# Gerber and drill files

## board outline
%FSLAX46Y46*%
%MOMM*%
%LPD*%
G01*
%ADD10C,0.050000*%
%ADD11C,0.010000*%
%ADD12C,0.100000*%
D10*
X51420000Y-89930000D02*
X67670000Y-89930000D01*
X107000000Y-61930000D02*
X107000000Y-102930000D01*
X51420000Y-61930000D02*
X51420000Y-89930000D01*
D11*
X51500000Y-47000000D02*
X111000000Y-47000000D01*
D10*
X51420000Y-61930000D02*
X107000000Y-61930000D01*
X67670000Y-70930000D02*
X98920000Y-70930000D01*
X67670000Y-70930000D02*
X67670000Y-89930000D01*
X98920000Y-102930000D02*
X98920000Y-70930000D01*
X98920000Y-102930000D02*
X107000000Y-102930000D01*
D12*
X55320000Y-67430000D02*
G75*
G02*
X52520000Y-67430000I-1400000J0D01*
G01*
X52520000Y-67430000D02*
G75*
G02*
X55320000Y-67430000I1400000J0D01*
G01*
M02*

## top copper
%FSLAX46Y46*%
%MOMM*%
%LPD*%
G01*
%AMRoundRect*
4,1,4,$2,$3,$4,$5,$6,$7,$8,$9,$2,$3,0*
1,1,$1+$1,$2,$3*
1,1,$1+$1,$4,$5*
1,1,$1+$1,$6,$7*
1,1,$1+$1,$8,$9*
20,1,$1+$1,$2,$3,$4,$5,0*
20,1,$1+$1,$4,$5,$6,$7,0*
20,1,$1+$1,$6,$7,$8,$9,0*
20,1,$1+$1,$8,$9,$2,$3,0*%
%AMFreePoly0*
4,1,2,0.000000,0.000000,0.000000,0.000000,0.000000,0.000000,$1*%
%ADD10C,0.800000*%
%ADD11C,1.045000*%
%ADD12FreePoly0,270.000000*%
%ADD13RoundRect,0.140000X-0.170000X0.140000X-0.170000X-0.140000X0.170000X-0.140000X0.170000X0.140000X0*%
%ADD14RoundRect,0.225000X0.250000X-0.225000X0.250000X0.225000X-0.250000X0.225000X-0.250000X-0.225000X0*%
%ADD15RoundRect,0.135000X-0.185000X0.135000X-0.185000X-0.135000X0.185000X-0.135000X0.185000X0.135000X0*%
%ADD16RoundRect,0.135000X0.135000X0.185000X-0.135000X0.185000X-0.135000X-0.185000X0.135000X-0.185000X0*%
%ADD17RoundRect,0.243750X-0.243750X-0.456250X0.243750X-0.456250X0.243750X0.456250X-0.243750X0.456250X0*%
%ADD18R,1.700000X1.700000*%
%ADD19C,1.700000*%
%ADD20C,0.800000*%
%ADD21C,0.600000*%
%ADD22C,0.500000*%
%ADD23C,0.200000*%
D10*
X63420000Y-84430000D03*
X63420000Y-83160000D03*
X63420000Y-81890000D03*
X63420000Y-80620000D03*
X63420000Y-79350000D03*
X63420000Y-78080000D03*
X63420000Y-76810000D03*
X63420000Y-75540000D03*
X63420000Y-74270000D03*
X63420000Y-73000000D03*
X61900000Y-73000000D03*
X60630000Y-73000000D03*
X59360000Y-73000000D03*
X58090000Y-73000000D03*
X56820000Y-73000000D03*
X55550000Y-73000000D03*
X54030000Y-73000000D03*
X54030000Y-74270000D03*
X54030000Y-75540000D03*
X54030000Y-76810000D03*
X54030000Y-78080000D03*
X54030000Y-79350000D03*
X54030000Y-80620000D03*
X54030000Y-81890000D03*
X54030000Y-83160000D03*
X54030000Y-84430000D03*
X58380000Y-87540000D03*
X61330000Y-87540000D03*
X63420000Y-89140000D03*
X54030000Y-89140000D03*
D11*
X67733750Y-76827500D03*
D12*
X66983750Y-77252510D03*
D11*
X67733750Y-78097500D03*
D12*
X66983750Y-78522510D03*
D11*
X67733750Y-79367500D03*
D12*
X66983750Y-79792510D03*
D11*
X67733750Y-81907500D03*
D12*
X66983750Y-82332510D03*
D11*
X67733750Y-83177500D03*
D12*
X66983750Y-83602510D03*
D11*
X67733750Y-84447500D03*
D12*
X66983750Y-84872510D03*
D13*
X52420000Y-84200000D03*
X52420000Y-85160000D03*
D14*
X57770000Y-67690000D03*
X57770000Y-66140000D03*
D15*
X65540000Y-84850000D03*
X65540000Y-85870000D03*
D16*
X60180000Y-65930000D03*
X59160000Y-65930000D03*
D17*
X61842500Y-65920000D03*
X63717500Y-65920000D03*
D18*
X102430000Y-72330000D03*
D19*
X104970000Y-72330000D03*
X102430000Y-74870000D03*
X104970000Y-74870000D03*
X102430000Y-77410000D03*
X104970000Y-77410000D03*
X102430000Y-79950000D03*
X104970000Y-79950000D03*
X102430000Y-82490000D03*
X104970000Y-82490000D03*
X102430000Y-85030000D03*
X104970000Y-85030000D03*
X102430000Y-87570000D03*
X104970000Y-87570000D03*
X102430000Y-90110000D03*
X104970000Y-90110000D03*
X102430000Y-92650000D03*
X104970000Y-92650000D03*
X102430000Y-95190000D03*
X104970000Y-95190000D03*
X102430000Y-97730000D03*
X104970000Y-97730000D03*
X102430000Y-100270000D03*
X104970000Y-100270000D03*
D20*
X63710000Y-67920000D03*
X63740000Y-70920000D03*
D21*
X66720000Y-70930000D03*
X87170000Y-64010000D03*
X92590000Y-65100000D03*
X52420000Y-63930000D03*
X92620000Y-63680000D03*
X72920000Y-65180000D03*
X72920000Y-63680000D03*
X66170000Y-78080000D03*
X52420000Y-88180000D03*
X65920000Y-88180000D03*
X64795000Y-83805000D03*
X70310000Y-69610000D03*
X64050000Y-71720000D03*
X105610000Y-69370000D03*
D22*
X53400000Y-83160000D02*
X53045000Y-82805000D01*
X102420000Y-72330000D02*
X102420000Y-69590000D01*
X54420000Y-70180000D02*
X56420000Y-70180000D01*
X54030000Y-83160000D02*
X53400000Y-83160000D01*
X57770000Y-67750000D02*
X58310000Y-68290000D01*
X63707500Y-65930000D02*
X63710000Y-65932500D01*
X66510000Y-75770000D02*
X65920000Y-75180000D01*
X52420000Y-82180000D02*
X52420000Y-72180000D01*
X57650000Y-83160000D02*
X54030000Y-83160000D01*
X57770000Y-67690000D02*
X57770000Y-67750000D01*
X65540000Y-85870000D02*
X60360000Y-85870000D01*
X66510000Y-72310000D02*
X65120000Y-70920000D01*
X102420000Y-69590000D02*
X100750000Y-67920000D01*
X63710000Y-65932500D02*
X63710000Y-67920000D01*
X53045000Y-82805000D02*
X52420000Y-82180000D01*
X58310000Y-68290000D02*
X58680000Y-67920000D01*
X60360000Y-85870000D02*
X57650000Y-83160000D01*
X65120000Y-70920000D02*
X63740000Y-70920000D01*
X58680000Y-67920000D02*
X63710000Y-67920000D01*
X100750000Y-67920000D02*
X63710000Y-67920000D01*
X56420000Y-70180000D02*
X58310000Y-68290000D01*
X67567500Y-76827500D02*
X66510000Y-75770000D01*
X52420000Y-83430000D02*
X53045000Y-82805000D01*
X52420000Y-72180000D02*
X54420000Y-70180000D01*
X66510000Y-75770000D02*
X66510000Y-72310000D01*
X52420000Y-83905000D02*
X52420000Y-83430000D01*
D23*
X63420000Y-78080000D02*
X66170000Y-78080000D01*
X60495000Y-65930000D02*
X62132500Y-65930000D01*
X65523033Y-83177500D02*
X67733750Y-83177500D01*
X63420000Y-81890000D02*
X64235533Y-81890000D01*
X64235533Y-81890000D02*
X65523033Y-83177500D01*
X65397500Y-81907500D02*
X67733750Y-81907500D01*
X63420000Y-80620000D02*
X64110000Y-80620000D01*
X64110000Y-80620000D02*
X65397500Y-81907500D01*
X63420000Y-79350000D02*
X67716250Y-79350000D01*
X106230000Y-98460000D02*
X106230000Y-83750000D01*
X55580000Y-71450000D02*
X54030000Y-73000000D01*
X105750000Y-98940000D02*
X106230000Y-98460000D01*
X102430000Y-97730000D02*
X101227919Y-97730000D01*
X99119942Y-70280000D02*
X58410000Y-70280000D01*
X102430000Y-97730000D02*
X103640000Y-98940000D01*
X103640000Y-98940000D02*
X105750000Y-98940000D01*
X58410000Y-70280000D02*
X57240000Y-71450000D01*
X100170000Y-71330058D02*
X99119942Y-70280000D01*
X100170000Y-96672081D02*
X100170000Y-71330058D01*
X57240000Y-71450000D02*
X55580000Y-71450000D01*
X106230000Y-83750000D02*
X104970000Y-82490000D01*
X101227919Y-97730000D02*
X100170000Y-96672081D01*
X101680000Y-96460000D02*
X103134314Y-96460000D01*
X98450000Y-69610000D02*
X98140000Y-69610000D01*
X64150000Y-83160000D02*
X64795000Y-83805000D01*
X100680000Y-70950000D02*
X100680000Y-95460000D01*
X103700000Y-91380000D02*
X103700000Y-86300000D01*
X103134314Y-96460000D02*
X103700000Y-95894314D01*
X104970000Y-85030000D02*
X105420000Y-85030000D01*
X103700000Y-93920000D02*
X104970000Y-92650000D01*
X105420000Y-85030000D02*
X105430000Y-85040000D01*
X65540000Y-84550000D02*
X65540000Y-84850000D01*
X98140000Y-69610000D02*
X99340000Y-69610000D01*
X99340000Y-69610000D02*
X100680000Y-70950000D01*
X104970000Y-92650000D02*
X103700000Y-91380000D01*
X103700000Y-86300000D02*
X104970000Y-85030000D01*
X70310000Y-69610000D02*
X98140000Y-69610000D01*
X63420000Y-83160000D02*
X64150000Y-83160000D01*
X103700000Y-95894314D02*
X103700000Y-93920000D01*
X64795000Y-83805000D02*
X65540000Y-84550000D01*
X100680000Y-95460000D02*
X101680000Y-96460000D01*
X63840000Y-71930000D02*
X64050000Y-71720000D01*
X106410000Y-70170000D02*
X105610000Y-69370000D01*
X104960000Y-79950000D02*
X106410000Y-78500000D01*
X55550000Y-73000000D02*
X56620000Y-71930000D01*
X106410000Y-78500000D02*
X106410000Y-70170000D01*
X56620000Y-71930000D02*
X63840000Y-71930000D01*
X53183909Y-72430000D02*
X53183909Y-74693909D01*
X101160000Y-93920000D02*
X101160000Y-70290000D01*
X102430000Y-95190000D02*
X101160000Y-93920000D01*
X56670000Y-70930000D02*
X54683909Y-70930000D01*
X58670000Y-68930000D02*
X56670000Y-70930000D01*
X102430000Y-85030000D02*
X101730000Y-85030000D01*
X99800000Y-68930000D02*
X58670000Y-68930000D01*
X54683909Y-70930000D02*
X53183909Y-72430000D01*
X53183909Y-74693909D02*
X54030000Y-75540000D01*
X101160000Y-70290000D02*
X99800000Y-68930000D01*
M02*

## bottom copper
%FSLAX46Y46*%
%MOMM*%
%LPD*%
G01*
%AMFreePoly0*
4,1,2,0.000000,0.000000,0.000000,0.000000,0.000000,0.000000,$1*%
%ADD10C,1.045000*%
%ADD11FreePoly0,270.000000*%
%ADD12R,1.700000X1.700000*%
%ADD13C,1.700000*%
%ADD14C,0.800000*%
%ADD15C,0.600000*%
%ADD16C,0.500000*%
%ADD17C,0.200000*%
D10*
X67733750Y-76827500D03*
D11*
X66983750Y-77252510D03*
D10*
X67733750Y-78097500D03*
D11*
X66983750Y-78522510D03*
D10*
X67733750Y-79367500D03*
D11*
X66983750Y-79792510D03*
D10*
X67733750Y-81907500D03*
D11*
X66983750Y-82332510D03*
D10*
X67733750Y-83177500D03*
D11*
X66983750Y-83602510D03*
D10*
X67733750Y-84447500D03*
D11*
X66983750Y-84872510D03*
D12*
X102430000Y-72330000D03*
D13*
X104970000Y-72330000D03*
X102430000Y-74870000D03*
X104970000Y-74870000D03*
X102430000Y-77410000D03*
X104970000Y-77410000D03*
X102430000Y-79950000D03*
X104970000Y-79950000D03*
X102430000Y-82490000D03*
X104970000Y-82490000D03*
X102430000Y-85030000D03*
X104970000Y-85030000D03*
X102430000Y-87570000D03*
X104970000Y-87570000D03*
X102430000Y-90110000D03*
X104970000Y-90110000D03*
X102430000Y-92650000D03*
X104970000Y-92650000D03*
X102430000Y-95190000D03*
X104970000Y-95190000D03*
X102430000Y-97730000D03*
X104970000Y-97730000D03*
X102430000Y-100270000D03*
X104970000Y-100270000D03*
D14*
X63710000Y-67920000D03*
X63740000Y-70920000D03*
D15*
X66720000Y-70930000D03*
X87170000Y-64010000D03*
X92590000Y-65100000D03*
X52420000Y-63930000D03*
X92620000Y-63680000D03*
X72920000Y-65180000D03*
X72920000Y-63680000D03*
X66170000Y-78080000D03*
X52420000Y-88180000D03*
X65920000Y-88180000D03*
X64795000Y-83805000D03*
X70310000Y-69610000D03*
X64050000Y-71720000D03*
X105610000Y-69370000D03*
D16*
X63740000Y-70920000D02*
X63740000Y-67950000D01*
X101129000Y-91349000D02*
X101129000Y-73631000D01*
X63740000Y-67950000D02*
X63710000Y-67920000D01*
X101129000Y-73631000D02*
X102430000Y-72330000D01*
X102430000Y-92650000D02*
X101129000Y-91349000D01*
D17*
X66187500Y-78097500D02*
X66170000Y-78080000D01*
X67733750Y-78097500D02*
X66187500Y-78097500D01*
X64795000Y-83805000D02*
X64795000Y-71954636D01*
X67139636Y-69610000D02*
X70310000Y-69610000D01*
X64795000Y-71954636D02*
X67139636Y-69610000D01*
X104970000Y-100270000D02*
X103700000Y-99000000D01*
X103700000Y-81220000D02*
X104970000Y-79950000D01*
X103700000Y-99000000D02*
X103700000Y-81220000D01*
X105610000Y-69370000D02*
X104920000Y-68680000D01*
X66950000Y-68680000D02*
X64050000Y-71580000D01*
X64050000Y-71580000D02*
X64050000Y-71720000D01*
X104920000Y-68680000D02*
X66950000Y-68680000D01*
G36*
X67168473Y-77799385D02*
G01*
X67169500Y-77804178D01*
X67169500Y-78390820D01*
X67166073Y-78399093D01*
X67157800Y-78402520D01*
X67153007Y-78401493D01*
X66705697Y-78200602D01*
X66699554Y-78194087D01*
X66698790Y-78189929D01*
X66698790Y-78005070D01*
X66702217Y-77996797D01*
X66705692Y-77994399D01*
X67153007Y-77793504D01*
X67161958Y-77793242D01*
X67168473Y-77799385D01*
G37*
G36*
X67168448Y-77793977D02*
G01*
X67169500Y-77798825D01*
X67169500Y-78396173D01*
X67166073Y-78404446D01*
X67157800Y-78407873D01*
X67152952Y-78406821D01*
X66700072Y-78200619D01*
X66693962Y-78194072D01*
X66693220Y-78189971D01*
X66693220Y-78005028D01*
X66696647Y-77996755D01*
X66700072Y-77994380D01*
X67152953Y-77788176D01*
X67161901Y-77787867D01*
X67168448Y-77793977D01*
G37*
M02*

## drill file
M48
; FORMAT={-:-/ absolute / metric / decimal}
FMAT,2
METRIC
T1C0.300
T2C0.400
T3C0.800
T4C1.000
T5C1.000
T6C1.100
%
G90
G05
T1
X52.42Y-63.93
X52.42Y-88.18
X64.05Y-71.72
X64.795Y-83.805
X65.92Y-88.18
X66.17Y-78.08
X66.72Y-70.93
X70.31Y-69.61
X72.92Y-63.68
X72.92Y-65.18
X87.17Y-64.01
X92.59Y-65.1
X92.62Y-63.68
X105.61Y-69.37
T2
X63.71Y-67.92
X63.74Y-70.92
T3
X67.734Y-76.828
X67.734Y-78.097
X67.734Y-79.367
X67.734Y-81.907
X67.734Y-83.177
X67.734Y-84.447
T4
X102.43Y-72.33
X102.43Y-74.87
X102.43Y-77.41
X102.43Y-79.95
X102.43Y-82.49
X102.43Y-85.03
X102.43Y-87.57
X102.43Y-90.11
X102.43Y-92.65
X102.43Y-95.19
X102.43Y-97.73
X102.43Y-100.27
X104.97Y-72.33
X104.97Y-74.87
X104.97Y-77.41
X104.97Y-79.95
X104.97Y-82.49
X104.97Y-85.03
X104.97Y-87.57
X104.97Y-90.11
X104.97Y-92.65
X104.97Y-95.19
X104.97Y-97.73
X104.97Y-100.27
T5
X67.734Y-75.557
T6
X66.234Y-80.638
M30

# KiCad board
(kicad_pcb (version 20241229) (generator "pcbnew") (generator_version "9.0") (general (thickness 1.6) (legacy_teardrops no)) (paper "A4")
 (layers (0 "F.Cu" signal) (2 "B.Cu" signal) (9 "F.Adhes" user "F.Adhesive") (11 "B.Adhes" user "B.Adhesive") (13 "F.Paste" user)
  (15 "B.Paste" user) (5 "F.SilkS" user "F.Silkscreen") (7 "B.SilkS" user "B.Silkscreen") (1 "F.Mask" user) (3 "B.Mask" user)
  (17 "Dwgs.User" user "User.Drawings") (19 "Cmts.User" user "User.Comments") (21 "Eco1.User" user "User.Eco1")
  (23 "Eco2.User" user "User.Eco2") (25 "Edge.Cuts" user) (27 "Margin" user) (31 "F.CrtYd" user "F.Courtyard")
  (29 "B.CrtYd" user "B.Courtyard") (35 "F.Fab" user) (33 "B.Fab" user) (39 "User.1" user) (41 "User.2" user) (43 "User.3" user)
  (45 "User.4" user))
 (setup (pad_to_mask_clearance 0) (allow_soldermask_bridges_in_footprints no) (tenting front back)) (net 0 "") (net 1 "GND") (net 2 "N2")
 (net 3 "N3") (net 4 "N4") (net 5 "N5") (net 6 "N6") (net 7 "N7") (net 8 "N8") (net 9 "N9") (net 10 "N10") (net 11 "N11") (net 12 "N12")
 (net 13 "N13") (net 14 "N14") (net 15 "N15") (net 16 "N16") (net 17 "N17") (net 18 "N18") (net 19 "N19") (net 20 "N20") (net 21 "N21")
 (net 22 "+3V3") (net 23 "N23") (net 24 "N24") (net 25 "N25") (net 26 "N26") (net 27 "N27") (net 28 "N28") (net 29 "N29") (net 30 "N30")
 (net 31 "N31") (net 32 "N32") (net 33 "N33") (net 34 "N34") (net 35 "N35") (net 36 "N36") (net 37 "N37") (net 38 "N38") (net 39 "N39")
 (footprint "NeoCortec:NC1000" (layer "F.Cu") (at 63.42 84.43 180)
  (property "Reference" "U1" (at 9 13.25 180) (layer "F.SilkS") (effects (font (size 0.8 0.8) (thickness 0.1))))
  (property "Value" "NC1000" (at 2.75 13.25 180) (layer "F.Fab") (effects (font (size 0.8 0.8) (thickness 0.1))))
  (pad "1" smd circle (at 0 0 180) (size 0.8 0.8) (layers "F.Cu" "F.Mask" "F.Paste") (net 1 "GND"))
  (pad "2" smd circle (at 0 1.27 180) (size 0.8 0.8) (layers "F.Cu" "F.Mask" "F.Paste") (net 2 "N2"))
  (pad "3" smd circle (at 0 2.54 180) (size 0.8 0.8) (layers "F.Cu" "F.Mask" "F.Paste") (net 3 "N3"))
  (pad "4" smd circle (at 0 3.81 180) (size 0.8 0.8) (layers "F.Cu" "F.Mask" "F.Paste") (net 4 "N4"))
  (pad "5" smd circle (at 0 5.08 180) (size 0.8 0.8) (layers "F.Cu" "F.Mask" "F.Paste") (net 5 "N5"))
  (pad "6" smd circle (at 0 6.35 180) (size 0.8 0.8) (layers "F.Cu" "F.Mask" "F.Paste") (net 1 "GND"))
  (pad "7" smd circle (at 0 7.62 180) (size 0.8 0.8) (layers "F.Cu" "F.Mask" "F.Paste") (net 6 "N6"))
  (pad "8" smd circle (at 0 8.89 180) (size 0.8 0.8) (layers "F.Cu" "F.Mask" "F.Paste") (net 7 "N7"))
  (pad "9" smd circle (at 0 10.16 180) (size 0.8 0.8) (layers "F.Cu" "F.Mask" "F.Paste") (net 1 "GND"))
  (pad "10" smd circle (at 0 11.43 180) (size 0.8 0.8) (layers "F.Cu" "F.Mask" "F.Paste") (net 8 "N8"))
  (pad "11" smd circle (at 1.52 11.43 180) (size 0.8 0.8) (layers "F.Cu" "F.Mask" "F.Paste") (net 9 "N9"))
  (pad "12" smd circle (at 2.79 11.43 180) (size 0.8 0.8) (layers "F.Cu" "F.Mask" "F.Paste") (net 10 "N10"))
  (pad "13" smd circle (at 4.06 11.43 180) (size 0.8 0.8) (layers "F.Cu" "F.Mask" "F.Paste") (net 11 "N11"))
  (pad "14" smd circle (at 5.33 11.43 180) (size 0.8 0.8) (layers "F.Cu" "F.Mask" "F.Paste") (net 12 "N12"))
  (pad "15" smd circle (at 6.6 11.43 180) (size 0.8 0.8) (layers "F.Cu" "F.Mask" "F.Paste") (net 1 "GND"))
  (pad "16" smd circle (at 7.87 11.43 180) (size 0.8 0.8) (layers "F.Cu" "F.Mask" "F.Paste") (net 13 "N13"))
  (pad "17" smd circle (at 9.39 11.43 180) (size 0.8 0.8) (layers "F.Cu" "F.Mask" "F.Paste") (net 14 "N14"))
  (pad "18" smd circle (at 9.39 10.16 180) (size 0.8 0.8) (layers "F.Cu" "F.Mask" "F.Paste") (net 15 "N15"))
  (pad "19" smd circle (at 9.39 8.89 180) (size 0.8 0.8) (layers "F.Cu" "F.Mask" "F.Paste") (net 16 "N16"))
  (pad "20" smd circle (at 9.39 7.62 180) (size 0.8 0.8) (layers "F.Cu" "F.Mask" "F.Paste") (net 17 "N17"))
  (pad "21" smd circle (at 9.39 6.35 180) (size 0.8 0.8) (layers "F.Cu" "F.Mask" "F.Paste") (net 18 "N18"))
  (pad "22" smd circle (at 9.39 5.08 180) (size 0.8 0.8) (layers "F.Cu" "F.Mask" "F.Paste") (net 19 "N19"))
  (pad "23" smd circle (at 9.39 3.81 180) (size 0.8 0.8) (layers "F.Cu" "F.Mask" "F.Paste") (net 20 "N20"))
  (pad "24" smd circle (at 9.39 2.54 180) (size 0.8 0.8) (layers "F.Cu" "F.Mask" "F.Paste") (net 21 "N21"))
  (pad "25" smd circle (at 9.39 1.27 180) (size 0.8 0.8) (layers "F.Cu" "F.Mask" "F.Paste") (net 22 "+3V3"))
  (pad "26" smd circle (at 9.39 0 180) (size 0.8 0.8) (layers "F.Cu" "F.Mask" "F.Paste") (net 1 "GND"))
  (pad "27" smd circle (at 5.04 -3.11 180) (size 0.8 0.8) (layers "F.Cu" "F.Mask" "F.Paste") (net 1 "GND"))
  (pad "28" smd circle (at 2.09 -3.11 180) (size 0.8 0.8) (layers "F.Cu" "F.Mask" "F.Paste") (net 1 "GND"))
  (pad "29" smd circle (at 0 -4.71 180) (size 0.8 0.8) (layers "F.Cu" "F.Mask" "F.Paste"))
  (pad "30" smd circle (at 9.39 -4.71 180) (size 0.8 0.8) (layers "F.Cu" "F.Mask" "F.Paste")))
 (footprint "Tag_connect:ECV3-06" (layer "F.Cu") (at 67.73375 76.8275 -90)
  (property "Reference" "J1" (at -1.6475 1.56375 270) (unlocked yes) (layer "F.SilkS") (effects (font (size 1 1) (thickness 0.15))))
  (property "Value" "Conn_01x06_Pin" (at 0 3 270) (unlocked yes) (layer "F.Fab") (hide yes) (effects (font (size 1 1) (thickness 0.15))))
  (pad "" np_thru_hole circle (at -1.27 0 270) (size 1 1) (drill 1) (layers "*.Cu" "*.Mask"))
  (pad "" np_thru_hole circle (at 3.81 1.5 270) (size 1.1 1.1) (drill 1.1) (layers "*.Cu" "*.Mask"))
  (pad "1" thru_hole circle (at 0 0 270) (size 1.045 1.045) (drill 0.8) (layers "*.Cu" "*.Mask") (remove_unused_layers no) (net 22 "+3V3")
   (solder_paste_margin -2147.483637))
  (pad "1" smd custom (at 0.42501 0.75 270) (size 0.000001 0.000001) (layers "F.Cu" "F.Mask") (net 22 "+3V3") (solder_mask_margin 0.000001)
   (options (clearance outline) (anchor circle)) (primitives))
  (pad "1" smd custom (at 0.42501 0.75 270) (size 0.000001 0.000001) (layers "B.Cu" "B.Mask") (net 22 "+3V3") (solder_mask_margin 0.000001)
   (options (clearance outline) (anchor circle)) (primitives))
  (pad "2" thru_hole circle (at 1.27 0 270) (size 1.045 1.045) (drill 0.8) (layers "*.Cu" "*.Mask") (remove_unused_layers no) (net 1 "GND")
   (solder_paste_margin -2147.483637)
   (teardrops (best_length_ratio 0.5) (max_length 1) (best_width_ratio 1) (max_width 2) (curved_edges no) (filter_ratio 0.9) (enabled yes)
    (allow_two_segments yes) (prefer_zone_connections yes)))
  (pad "2" smd custom (at 1.69501 0.75 270) (size 0.000001 0.000001) (layers "F.Cu" "F.Mask") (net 1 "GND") (solder_mask_margin 0.000001)
   (options (clearance outline) (anchor circle)) (primitives))
  (pad "2" smd custom (at 1.69501 0.75 270) (size 0.000001 0.000001) (layers "B.Cu" "B.Mask") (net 1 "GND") (solder_mask_margin 0.000001)
   (options (clearance outline) (anchor circle)) (primitives))
  (pad "3" thru_hole circle (at 2.54 0 270) (size 1.045 1.045) (drill 0.8) (layers "*.Cu" "*.Mask") (remove_unused_layers no) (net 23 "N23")
   (solder_paste_margin -2147.483637))
  (pad "3" smd custom (at 2.96501 0.75 270) (size 0.000001 0.000001) (layers "F.Cu" "F.Mask") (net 23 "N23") (solder_mask_margin 0.000001)
   (options (clearance outline) (anchor circle)) (primitives))
  (pad "3" smd custom (at 2.96501 0.75 270) (size 0.000001 0.000001) (layers "B.Cu" "B.Mask") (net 23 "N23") (solder_mask_margin 0.000001)
   (options (clearance outline) (anchor circle)) (primitives))
  (pad "4" thru_hole circle (at 5.08 0 270) (size 1.045 1.045) (drill 0.8) (layers "*.Cu" "*.Mask") (remove_unused_layers no) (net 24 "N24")
   (solder_paste_margin -2147.483637))
  (pad "4" smd custom (at 5.50501 0.75 270) (size 0.000001 0.000001) (layers "F.Cu" "F.Mask") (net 24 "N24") (solder_mask_margin 0.000001)
   (options (clearance outline) (anchor circle)) (primitives))
  (pad "4" smd custom (at 5.50501 0.75 270) (size 0.000001 0.000001) (layers "B.Cu" "B.Mask") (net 24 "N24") (solder_mask_margin 0.000001)
   (options (clearance outline) (anchor circle)) (primitives))
  (pad "5" thru_hole circle (at 6.35 0 270) (size 1.045 1.045) (drill 0.8) (layers "*.Cu" "*.Mask") (remove_unused_layers no) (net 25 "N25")
   (solder_paste_margin -2147.483637))
  (pad "5" smd custom (at 6.77501 0.75 270) (size 0.000001 0.000001) (layers "F.Cu" "F.Mask") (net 25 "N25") (solder_mask_margin 0.000001)
   (options (clearance outline) (anchor circle)) (primitives))
  (pad "5" smd custom (at 6.77501 0.75 270) (size 0.000001 0.000001) (layers "B.Cu" "B.Mask") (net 25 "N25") (solder_mask_margin 0.000001)
   (options (clearance outline) (anchor circle)) (primitives))
  (pad "6" thru_hole circle (at 7.62 0 270) (size 1.045 1.045) (drill 0.8) (layers "*.Cu" "*.Mask") (remove_unused_layers no) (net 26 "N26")
   (solder_paste_margin -2147.483637))
  (pad "6" smd custom (at 8.04501 0.75 270) (size 0.000001 0.000001) (layers "F.Cu" "F.Mask") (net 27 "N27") (solder_mask_margin 0.000001)
   (options (clearance outline) (anchor circle)) (primitives))
  (pad "6" smd custom (at 8.04501 0.75 270) (size 0.000001 0.000001) (layers "B.Cu" "B.Mask") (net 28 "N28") (solder_mask_margin 0.000001)
   (options (clearance outline) (anchor circle)) (primitives)))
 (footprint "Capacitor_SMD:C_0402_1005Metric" (layer "F.Cu") (at 52.42 84.68 -90)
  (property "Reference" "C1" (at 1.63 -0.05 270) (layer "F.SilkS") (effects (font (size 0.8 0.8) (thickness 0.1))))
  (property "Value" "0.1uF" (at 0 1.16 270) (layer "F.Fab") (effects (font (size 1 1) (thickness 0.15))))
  (pad "1" smd roundrect (at -0.48 0 270) (size 0.56 0.62) (layers "F.Cu" "F.Mask" "F.Paste") (roundrect_rratio 0.25) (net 22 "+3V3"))
  (pad "2" smd roundrect (at 0.48 0 270) (size 0.56 0.62) (layers "F.Cu" "F.Mask" "F.Paste") (roundrect_rratio 0.25) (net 1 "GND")))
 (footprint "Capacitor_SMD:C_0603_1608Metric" (layer "F.Cu") (at 57.77 66.915 90)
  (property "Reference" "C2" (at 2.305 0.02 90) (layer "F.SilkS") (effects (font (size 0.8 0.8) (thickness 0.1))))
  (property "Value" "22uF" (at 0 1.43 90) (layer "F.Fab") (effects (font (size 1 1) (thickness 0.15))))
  (pad "1" smd roundrect (at -0.775 0 90) (size 0.9 0.95) (layers "F.Cu" "F.Mask" "F.Paste") (roundrect_rratio 0.25) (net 22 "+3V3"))
  (pad "2" smd roundrect (at 0.775 0 90) (size 0.9 0.95) (layers "F.Cu" "F.Mask" "F.Paste") (roundrect_rratio 0.25) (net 1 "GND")))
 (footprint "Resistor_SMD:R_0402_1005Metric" (layer "F.Cu") (at 65.54 85.36 -90)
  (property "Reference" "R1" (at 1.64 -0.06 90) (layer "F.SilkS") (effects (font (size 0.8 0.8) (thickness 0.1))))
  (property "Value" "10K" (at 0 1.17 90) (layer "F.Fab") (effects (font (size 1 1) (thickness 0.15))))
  (pad "1" smd roundrect (at -0.51 0 270) (size 0.54 0.64) (layers "F.Cu" "F.Mask" "F.Paste") (roundrect_rratio 0.25) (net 22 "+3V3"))
  (pad "2" smd roundrect (at 0.51 0 270) (size 0.54 0.64) (layers "F.Cu" "F.Mask" "F.Paste") (roundrect_rratio 0.25) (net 2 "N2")))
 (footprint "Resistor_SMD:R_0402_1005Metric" (layer "F.Cu") (at 59.67 65.93 180)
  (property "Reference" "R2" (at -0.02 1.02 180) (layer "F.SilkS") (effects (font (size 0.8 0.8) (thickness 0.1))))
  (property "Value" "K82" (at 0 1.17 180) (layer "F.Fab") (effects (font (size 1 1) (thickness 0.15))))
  (pad "1" smd roundrect (at -0.51 0 180) (size 0.54 0.64) (layers "F.Cu" "F.Mask" "F.Paste") (roundrect_rratio 0.25) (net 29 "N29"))
  (pad "2" smd roundrect (at 0.51 0 180) (size 0.54 0.64) (layers "F.Cu" "F.Mask" "F.Paste") (roundrect_rratio 0.25) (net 1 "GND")))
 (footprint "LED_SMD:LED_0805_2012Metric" (layer "F.Cu") (at 62.78 65.92)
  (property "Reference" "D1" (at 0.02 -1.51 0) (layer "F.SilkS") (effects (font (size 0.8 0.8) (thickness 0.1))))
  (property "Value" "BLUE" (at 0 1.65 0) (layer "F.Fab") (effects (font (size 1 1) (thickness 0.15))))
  (pad "1" smd roundrect (at -0.9375 0) (size 0.975 1.4) (layers "F.Cu" "F.Mask" "F.Paste") (roundrect_rratio 0.25) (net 29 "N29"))
  (pad "2" smd roundrect (at 0.9375 0) (size 0.975 1.4) (layers "F.Cu" "F.Mask" "F.Paste") (roundrect_rratio 0.25) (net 22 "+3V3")))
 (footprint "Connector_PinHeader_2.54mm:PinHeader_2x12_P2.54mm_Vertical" (layer "F.Cu") (at 102.43 72.33)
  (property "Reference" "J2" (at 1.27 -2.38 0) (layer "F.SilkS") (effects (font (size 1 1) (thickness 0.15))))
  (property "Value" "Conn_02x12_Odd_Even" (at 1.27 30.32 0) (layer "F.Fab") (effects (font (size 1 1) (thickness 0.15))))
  (pad "1" thru_hole rect (at 0 0) (size 1.7 1.7) (drill 1) (layers "*.Cu" "*.Mask") (remove_unused_layers no) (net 22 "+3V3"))
  (pad "2" thru_hole circle (at 2.54 0) (size 1.7 1.7) (drill 1) (layers "*.Cu" "*.Mask") (remove_unused_layers no) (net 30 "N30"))
  (pad "3" thru_hole circle (at 0 2.54) (size 1.7 1.7) (drill 1) (layers "*.Cu" "*.Mask") (remove_unused_layers no) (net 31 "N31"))
  (pad "4" thru_hole circle (at 2.54 2.54) (size 1.7 1.7) (drill 1) (layers "*.Cu" "*.Mask") (remove_unused_layers no) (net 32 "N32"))
  (pad "5" thru_hole circle (at 0 5.08) (size 1.7 1.7) (drill 1) (layers "*.Cu" "*.Mask") (remove_unused_layers no) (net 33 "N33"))
  (pad "6" thru_hole circle (at 2.54 5.08) (size 1.7 1.7) (drill 1) (layers "*.Cu" "*.Mask") (remove_unused_layers no) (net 1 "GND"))
  (pad "7" thru_hole circle (at 0 7.62) (size 1.7 1.7) (drill 1) (layers "*.Cu" "*.Mask") (remove_unused_layers no) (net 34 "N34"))
  (pad "8" thru_hole circle (at 2.54 7.62) (size 1.7 1.7) (drill 1) (layers "*.Cu" "*.Mask") (remove_unused_layers no) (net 13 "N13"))
  (pad "9" thru_hole circle (at 0 10.16) (size 1.7 1.7) (drill 1) (layers "*.Cu" "*.Mask") (remove_unused_layers no) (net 1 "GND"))
  (pad "10" thru_hole circle (at 2.54 10.16) (size 1.7 1.7) (drill 1) (layers "*.Cu" "*.Mask") (remove_unused_layers no) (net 14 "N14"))
  (pad "11" thru_hole circle (at 0 12.7) (size 1.7 1.7) (drill 1) (layers "*.Cu" "*.Mask") (remove_unused_layers no) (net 16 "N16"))
  (pad "12" thru_hole circle (at 2.54 12.7) (size 1.7 1.7) (drill 1) (layers "*.Cu" "*.Mask") (remove_unused_layers no) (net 2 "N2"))
  (pad "13" thru_hole circle (at 0 15.24) (size 1.7 1.7) (drill 1) (layers "*.Cu" "*.Mask") (remove_unused_layers no) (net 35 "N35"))
  (pad "14" thru_hole circle (at 2.54 15.24) (size 1.7 1.7) (drill 1) (layers "*.Cu" "*.Mask") (remove_unused_layers no) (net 1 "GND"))
  (pad "15" thru_hole circle (at 0 17.78) (size 1.7 1.7) (drill 1) (layers "*.Cu" "*.Mask") (remove_unused_layers no) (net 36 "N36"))
  (pad "16" thru_hole circle (at 2.54 17.78) (size 1.7 1.7) (drill 1) (layers "*.Cu" "*.Mask") (remove_unused_layers no) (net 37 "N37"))
  (pad "17" thru_hole circle (at 0 20.32) (size 1.7 1.7) (drill 1) (layers "*.Cu" "*.Mask") (remove_unused_layers no) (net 22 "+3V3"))
  (pad "18" thru_hole circle (at 2.54 20.32) (size 1.7 1.7) (drill 1) (layers "*.Cu" "*.Mask") (remove_unused_layers no) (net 2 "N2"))
  (pad "19" thru_hole circle (at 0 22.86) (size 1.7 1.7) (drill 1) (layers "*.Cu" "*.Mask") (remove_unused_layers no) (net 16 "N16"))
  (pad "20" thru_hole circle (at 2.54 22.86) (size 1.7 1.7) (drill 1) (layers "*.Cu" "*.Mask") (remove_unused_layers no) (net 1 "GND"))
  (pad "21" thru_hole circle (at 0 25.4) (size 1.7 1.7) (drill 1) (layers "*.Cu" "*.Mask") (remove_unused_layers no) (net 14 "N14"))
  (pad "22" thru_hole circle (at 2.54 25.4) (size 1.7 1.7) (drill 1) (layers "*.Cu" "*.Mask") (remove_unused_layers no) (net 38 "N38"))
  (pad "23" thru_hole circle (at 0 27.94) (size 1.7 1.7) (drill 1) (layers "*.Cu" "*.Mask") (remove_unused_layers no) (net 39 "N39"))
  (pad "24" thru_hole circle (at 2.54 27.94) (size 1.7 1.7) (drill 1) (layers "*.Cu" "*.Mask") (remove_unused_layers no) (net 13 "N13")))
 (gr_line (start 51.42 89.93) (end 67.67 89.93) (stroke (width 0.05) (type solid)) (layer "Edge.Cuts"))
 (gr_line (start 107 61.93) (end 107 102.93) (stroke (width 0.05) (type solid)) (layer "Edge.Cuts"))
 (gr_line (start 51.42 61.93) (end 51.42 89.93) (stroke (width 0.05) (type solid)) (layer "Edge.Cuts"))
 (gr_line (start 51.5 47) (end 111 47) (stroke (width 0.01) (type solid)) (locked yes) (layer "Edge.Cuts"))
 (gr_line (start 51.42 61.93) (end 107 61.93) (stroke (width 0.05) (type solid)) (layer "Edge.Cuts"))
 (gr_line (start 67.67 70.93) (end 98.92 70.93) (stroke (width 0.05) (type solid)) (layer "Edge.Cuts"))
 (gr_line (start 67.67 70.93) (end 67.67 89.93) (stroke (width 0.05) (type solid)) (layer "Edge.Cuts"))
 (gr_line (start 98.92 102.93) (end 98.92 70.93) (stroke (width 0.05) (type solid)) (layer "Edge.Cuts"))
 (gr_line (start 98.92 102.93) (end 107 102.93) (stroke (width 0.05) (type solid)) (layer "Edge.Cuts"))
 (gr_circle (center 53.92 67.43) (end 55.32 67.43) (stroke (width 0.1) (type solid)) (fill no) (layer "Edge.Cuts"))
 (segment (start 53.4 83.16) (end 53.045 82.805) (width 0.5) (layer "F.Cu") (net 22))
 (segment (start 102.42 72.33) (end 102.42 69.59) (width 0.5) (layer "F.Cu") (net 22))
 (segment (start 54.42 70.18) (end 56.42 70.18) (width 0.5) (layer "F.Cu") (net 22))
 (segment (start 54.03 83.16) (end 53.4 83.16) (width 0.5) (layer "F.Cu") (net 22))
 (segment (start 57.77 67.75) (end 58.31 68.29) (width 0.5) (layer "F.Cu") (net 22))
 (segment (start 63.7075 65.93) (end 63.71 65.9325) (width 0.5) (layer "F.Cu") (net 22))
 (segment (start 66.51 75.77) (end 65.92 75.18) (width 0.5) (layer "F.Cu") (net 22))
 (segment (start 52.42 82.18) (end 52.42 72.18) (width 0.5) (layer "F.Cu") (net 22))
 (segment (start 57.65 83.16) (end 54.03 83.16) (width 0.5) (layer "F.Cu") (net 22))
 (segment (start 57.77 67.69) (end 57.77 67.75) (width 0.5) (layer "F.Cu") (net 22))
 (segment (start 65.54 85.87) (end 60.36 85.87) (width 0.5) (layer "F.Cu") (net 22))
 (segment (start 66.51 72.31) (end 65.12 70.92) (width 0.5) (layer "F.Cu") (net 22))
 (segment (start 102.42 69.59) (end 100.75 67.92) (width 0.5) (layer "F.Cu") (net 22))
 (segment (start 63.71 65.9325) (end 63.71 67.92) (width 0.5) (layer "F.Cu") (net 22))
 (segment (start 53.045 82.805) (end 52.42 82.18) (width 0.5) (layer "F.Cu") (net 22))
 (segment (start 58.31 68.29) (end 58.68 67.92) (width 0.5) (layer "F.Cu") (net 22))
 (segment (start 60.36 85.87) (end 57.65 83.16) (width 0.5) (layer "F.Cu") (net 22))
 (segment (start 65.12 70.92) (end 63.74 70.92) (width 0.5) (layer "F.Cu") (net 22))
 (segment (start 58.68 67.92) (end 63.71 67.92) (width 0.5) (layer "F.Cu") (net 22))
 (segment (start 100.75 67.92) (end 63.71 67.92) (width 0.5) (layer "F.Cu") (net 22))
 (segment (start 56.42 70.18) (end 58.31 68.29) (width 0.5) (layer "F.Cu") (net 22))
 (segment (start 67.5675 76.8275) (end 66.51 75.77) (width 0.5) (layer "F.Cu") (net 22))
 (segment (start 52.42 83.43) (end 53.045 82.805) (width 0.5) (layer "F.Cu") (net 22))
 (segment (start 52.42 72.18) (end 54.42 70.18) (width 0.5) (layer "F.Cu") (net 22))
 (segment (start 66.51 75.77) (end 66.51 72.31) (width 0.5) (layer "F.Cu") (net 22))
 (segment (start 52.42 83.905) (end 52.42 83.43) (width 0.5) (layer "F.Cu") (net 22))
 (via (at 63.71 67.92) (size 0.8) (drill 0.4) (layers "F.Cu" "B.Cu") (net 22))
 (via (at 63.74 70.92) (size 0.8) (drill 0.4) (layers "F.Cu" "B.Cu") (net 22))
 (segment (start 63.74 70.92) (end 63.74 67.95) (width 0.5) (layer "B.Cu") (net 22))
 (segment (start 101.129 91.349) (end 101.129 73.631) (width 0.5) (layer "B.Cu") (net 22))
 (segment (start 63.74 67.95) (end 63.71 67.92) (width 0.5) (layer "B.Cu") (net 22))
 (segment (start 101.129 73.631) (end 102.43 72.33) (width 0.5) (layer "B.Cu") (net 22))
 (segment (start 102.43 92.65) (end 101.129 91.349) (width 0.5) (layer "B.Cu") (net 22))
 (segment (start 63.42 78.08) (end 66.17 78.08) (width 0.2) (layer "F.Cu") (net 1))
 (via (at 66.72 70.93) (size 0.6) (drill 0.3) (layers "F.Cu" "B.Cu") (free yes) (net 1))
 (via (at 87.17 64.01) (size 0.6) (drill 0.3) (layers "F.Cu" "B.Cu") (free yes) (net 1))
 (via (at 92.59 65.1) (size 0.6) (drill 0.3) (layers "F.Cu" "B.Cu") (free yes) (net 1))
 (via (at 52.42 63.93) (size 0.6) (drill 0.3) (layers "F.Cu" "B.Cu") (free yes) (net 1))
 (via (at 92.62 63.68) (size 0.6) (drill 0.3) (layers "F.Cu" "B.Cu") (free yes) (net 1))
 (via (at 72.92 65.18) (size 0.6) (drill 0.3) (layers "F.Cu" "B.Cu") (free yes) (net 1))
 (via (at 72.92 63.68) (size 0.6) (drill 0.3) (layers "F.Cu" "B.Cu") (free yes) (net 1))
 (via (at 66.17 78.08) (size 0.6) (drill 0.3) (layers "F.Cu" "B.Cu") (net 1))
 (via (at 52.42 88.18) (size 0.6) (drill 0.3) (layers "F.Cu" "B.Cu") (free yes) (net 1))
 (via (at 65.92 88.18) (size 0.6) (drill 0.3) (layers "F.Cu" "B.Cu") (free yes) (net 1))
 (segment (start 66.1875 78.0975) (end 66.17 78.08) (width 0.2) (layer "B.Cu") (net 1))
 (segment (start 67.73375 78.0975) (end 66.1875 78.0975) (width 0.2) (layer "B.Cu") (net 1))
 (segment (start 60.495 65.93) (end 62.1325 65.93) (width 0.2) (layer "F.Cu") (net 29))
 (segment (start 65.523033 83.1775) (end 67.73375 83.1775) (width 0.2) (layer "F.Cu") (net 25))
 (segment (start 63.42 81.89) (end 64.235533 81.89) (width 0.2) (layer "F.Cu") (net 25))
 (segment (start 64.235533 81.89) (end 65.523033 83.1775) (width 0.2) (layer "F.Cu") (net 25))
 (segment (start 65.3975 81.9075) (end 67.73375 81.9075) (width 0.2) (layer "F.Cu") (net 24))
 (segment (start 63.42 80.62) (end 64.11 80.62) (width 0.2) (layer "F.Cu") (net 24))
 (segment (start 64.11 80.62) (end 65.3975 81.9075) (width 0.2) (layer "F.Cu") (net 24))
 (segment (start 63.42 79.35) (end 67.71625 79.35) (width 0.2) (layer "F.Cu") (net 23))
 (segment (start 106.23 98.46) (end 106.23 83.75) (width 0.2) (layer "F.Cu") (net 14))
 (segment (start 55.58 71.45) (end 54.03 73) (width 0.2) (layer "F.Cu") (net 14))
 (segment (start 105.75 98.94) (end 106.23 98.46) (width 0.2) (layer "F.Cu") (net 14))
 (segment (start 102.43 97.73) (end 101.227919 97.73) (width 0.2) (layer "F.Cu") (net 14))
 (segment (start 99.119942 70.28) (end 58.41 70.28) (width 0.2) (layer "F.Cu") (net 14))
 (segment (start 102.43 97.73) (end 103.64 98.94) (width 0.2) (layer "F.Cu") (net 14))
 (segment (start 103.64 98.94) (end 105.75 98.94) (width 0.2) (layer "F.Cu") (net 14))
 (segment (start 58.41 70.28) (end 57.24 71.45) (width 0.2) (layer "F.Cu") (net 14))
 (segment (start 100.17 71.330058) (end 99.119942 70.28) (width 0.2) (layer "F.Cu") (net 14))
 (segment (start 100.17 96.672081) (end 100.17 71.330058) (width 0.2) (layer "F.Cu") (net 14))
 (segment (start 57.24 71.45) (end 55.58 71.45) (width 0.2) (layer "F.Cu") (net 14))
 (segment (start 106.23 83.75) (end 104.97 82.49) (width 0.2) (layer "F.Cu") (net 14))
 (segment (start 101.227919 97.73) (end 100.17 96.672081) (width 0.2) (layer "F.Cu") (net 14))
 (segment (start 101.68 96.46) (end 103.134314 96.46) (width 0.2) (layer "F.Cu") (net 2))
 (segment (start 98.45 69.61) (end 98.14 69.61) (width 0.2) (layer "F.Cu") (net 2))
 (segment (start 64.15 83.16) (end 64.795 83.805) (width 0.2) (layer "F.Cu") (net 2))
 (segment (start 100.68 70.95) (end 100.68 95.46) (width 0.2) (layer "F.Cu") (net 2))
 (segment (start 103.7 91.38) (end 103.7 86.3) (width 0.2) (layer "F.Cu") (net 2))
 (segment (start 103.134314 96.46) (end 103.7 95.894314) (width 0.2) (layer "F.Cu") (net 2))
 (segment (start 104.97 85.03) (end 105.42 85.03) (width 0.2) (layer "F.Cu") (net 2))
 (segment (start 103.7 93.92) (end 104.97 92.65) (width 0.2) (layer "F.Cu") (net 2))
 (segment (start 105.42 85.03) (end 105.43 85.04) (width 0.2) (layer "F.Cu") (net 2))
 (segment (start 65.54 84.55) (end 65.54 84.85) (width 0.2) (layer "F.Cu") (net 2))
 (segment (start 98.14 69.61) (end 99.34 69.61) (width 0.2) (layer "F.Cu") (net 2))
 (segment (start 99.34 69.61) (end 100.68 70.95) (width 0.2) (layer "F.Cu") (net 2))
 (segment (start 104.97 92.65) (end 103.7 91.38) (width 0.2) (layer "F.Cu") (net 2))
 (segment (start 103.7 86.3) (end 104.97 85.03) (width 0.2) (layer "F.Cu") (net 2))
 (segment (start 70.31 69.61) (end 98.14 69.61) (width 0.2) (layer "F.Cu") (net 2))
 (segment (start 63.42 83.16) (end 64.15 83.16) (width 0.2) (layer "F.Cu") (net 2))
 (segment (start 103.7 95.894314) (end 103.7 93.92) (width 0.2) (layer "F.Cu") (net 2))
 (segment (start 64.795 83.805) (end 65.54 84.55) (width 0.2) (layer "F.Cu") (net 2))
 (segment (start 100.68 95.46) (end 101.68 96.46) (width 0.2) (layer "F.Cu") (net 2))
 (via (at 64.795 83.805) (size 0.6) (drill 0.3) (layers "F.Cu" "B.Cu") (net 2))
 (via (at 70.31 69.61) (size 0.6) (drill 0.3) (layers "F.Cu" "B.Cu") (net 2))
 (segment (start 64.795 83.805) (end 64.795 71.954636) (width 0.2) (layer "B.Cu") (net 2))
 (segment (start 67.139636 69.61) (end 70.31 69.61) (width 0.2) (layer "B.Cu") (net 2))
 (segment (start 64.795 71.954636) (end 67.139636 69.61) (width 0.2) (layer "B.Cu") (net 2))
 (segment (start 63.84 71.93) (end 64.05 71.72) (width 0.2) (layer "F.Cu") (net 13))
 (segment (start 106.41 70.17) (end 105.61 69.37) (width 0.2) (layer "F.Cu") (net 13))
 (segment (start 104.96 79.95) (end 106.41 78.5) (width 0.2) (layer "F.Cu") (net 13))
 (segment (start 55.55 73) (end 56.62 71.93) (width 0.2) (layer "F.Cu") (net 13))
 (segment (start 106.41 78.5) (end 106.41 70.17) (width 0.2) (layer "F.Cu") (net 13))
 (segment (start 56.62 71.93) (end 63.84 71.93) (width 0.2) (layer "F.Cu") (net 13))
 (via (at 64.05 71.72) (size 0.6) (drill 0.3) (layers "F.Cu" "B.Cu") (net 13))
 (via (at 105.61 69.37) (size 0.6) (drill 0.3) (layers "F.Cu" "B.Cu") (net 13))
 (segment (start 104.97 100.27) (end 103.7 99) (width 0.2) (layer "B.Cu") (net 13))
 (segment (start 103.7 81.22) (end 104.97 79.95) (width 0.2) (layer "B.Cu") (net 13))
 (segment (start 103.7 99) (end 103.7 81.22) (width 0.2) (layer "B.Cu") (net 13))
 (segment (start 105.61 69.37) (end 104.92 68.68) (width 0.2) (layer "B.Cu") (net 13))
 (segment (start 66.95 68.68) (end 64.05 71.58) (width 0.2) (layer "B.Cu") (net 13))
 (segment (start 64.05 71.58) (end 64.05 71.72) (width 0.2) (layer "B.Cu") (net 13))
 (segment (start 104.92 68.68) (end 66.95 68.68) (width 0.2) (layer "B.Cu") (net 13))
 (segment (start 53.183909 72.43) (end 53.183909 74.693909) (width 0.2) (layer "F.Cu") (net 16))
 (segment (start 101.16 93.92) (end 101.16 70.29) (width 0.2) (layer "F.Cu") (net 16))
 (segment (start 102.43 95.19) (end 101.16 93.92) (width 0.2) (layer "F.Cu") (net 16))
 (segment (start 56.67 70.93) (end 54.683909 70.93) (width 0.2) (layer "F.Cu") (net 16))
 (segment (start 58.67 68.93) (end 56.67 70.93) (width 0.2) (layer "F.Cu") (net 16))
 (segment (start 102.43 85.03) (end 101.73 85.03) (width 0.2) (layer "F.Cu") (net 16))
 (segment (start 99.8 68.93) (end 58.67 68.93) (width 0.2) (layer "F.Cu") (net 16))
 (segment (start 54.683909 70.93) (end 53.183909 72.43) (width 0.2) (layer "F.Cu") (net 16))
 (segment (start 53.183909 74.693909) (end 54.03 75.54) (width 0.2) (layer "F.Cu") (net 16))
 (segment (start 101.16 70.29) (end 99.8 68.93) (width 0.2) (layer "F.Cu") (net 16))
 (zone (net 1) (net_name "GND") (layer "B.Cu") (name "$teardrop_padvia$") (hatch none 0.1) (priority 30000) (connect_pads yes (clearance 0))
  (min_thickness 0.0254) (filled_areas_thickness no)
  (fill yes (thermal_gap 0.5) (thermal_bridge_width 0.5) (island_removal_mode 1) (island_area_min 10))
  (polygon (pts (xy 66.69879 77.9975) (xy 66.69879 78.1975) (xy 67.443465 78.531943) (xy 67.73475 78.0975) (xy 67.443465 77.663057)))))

